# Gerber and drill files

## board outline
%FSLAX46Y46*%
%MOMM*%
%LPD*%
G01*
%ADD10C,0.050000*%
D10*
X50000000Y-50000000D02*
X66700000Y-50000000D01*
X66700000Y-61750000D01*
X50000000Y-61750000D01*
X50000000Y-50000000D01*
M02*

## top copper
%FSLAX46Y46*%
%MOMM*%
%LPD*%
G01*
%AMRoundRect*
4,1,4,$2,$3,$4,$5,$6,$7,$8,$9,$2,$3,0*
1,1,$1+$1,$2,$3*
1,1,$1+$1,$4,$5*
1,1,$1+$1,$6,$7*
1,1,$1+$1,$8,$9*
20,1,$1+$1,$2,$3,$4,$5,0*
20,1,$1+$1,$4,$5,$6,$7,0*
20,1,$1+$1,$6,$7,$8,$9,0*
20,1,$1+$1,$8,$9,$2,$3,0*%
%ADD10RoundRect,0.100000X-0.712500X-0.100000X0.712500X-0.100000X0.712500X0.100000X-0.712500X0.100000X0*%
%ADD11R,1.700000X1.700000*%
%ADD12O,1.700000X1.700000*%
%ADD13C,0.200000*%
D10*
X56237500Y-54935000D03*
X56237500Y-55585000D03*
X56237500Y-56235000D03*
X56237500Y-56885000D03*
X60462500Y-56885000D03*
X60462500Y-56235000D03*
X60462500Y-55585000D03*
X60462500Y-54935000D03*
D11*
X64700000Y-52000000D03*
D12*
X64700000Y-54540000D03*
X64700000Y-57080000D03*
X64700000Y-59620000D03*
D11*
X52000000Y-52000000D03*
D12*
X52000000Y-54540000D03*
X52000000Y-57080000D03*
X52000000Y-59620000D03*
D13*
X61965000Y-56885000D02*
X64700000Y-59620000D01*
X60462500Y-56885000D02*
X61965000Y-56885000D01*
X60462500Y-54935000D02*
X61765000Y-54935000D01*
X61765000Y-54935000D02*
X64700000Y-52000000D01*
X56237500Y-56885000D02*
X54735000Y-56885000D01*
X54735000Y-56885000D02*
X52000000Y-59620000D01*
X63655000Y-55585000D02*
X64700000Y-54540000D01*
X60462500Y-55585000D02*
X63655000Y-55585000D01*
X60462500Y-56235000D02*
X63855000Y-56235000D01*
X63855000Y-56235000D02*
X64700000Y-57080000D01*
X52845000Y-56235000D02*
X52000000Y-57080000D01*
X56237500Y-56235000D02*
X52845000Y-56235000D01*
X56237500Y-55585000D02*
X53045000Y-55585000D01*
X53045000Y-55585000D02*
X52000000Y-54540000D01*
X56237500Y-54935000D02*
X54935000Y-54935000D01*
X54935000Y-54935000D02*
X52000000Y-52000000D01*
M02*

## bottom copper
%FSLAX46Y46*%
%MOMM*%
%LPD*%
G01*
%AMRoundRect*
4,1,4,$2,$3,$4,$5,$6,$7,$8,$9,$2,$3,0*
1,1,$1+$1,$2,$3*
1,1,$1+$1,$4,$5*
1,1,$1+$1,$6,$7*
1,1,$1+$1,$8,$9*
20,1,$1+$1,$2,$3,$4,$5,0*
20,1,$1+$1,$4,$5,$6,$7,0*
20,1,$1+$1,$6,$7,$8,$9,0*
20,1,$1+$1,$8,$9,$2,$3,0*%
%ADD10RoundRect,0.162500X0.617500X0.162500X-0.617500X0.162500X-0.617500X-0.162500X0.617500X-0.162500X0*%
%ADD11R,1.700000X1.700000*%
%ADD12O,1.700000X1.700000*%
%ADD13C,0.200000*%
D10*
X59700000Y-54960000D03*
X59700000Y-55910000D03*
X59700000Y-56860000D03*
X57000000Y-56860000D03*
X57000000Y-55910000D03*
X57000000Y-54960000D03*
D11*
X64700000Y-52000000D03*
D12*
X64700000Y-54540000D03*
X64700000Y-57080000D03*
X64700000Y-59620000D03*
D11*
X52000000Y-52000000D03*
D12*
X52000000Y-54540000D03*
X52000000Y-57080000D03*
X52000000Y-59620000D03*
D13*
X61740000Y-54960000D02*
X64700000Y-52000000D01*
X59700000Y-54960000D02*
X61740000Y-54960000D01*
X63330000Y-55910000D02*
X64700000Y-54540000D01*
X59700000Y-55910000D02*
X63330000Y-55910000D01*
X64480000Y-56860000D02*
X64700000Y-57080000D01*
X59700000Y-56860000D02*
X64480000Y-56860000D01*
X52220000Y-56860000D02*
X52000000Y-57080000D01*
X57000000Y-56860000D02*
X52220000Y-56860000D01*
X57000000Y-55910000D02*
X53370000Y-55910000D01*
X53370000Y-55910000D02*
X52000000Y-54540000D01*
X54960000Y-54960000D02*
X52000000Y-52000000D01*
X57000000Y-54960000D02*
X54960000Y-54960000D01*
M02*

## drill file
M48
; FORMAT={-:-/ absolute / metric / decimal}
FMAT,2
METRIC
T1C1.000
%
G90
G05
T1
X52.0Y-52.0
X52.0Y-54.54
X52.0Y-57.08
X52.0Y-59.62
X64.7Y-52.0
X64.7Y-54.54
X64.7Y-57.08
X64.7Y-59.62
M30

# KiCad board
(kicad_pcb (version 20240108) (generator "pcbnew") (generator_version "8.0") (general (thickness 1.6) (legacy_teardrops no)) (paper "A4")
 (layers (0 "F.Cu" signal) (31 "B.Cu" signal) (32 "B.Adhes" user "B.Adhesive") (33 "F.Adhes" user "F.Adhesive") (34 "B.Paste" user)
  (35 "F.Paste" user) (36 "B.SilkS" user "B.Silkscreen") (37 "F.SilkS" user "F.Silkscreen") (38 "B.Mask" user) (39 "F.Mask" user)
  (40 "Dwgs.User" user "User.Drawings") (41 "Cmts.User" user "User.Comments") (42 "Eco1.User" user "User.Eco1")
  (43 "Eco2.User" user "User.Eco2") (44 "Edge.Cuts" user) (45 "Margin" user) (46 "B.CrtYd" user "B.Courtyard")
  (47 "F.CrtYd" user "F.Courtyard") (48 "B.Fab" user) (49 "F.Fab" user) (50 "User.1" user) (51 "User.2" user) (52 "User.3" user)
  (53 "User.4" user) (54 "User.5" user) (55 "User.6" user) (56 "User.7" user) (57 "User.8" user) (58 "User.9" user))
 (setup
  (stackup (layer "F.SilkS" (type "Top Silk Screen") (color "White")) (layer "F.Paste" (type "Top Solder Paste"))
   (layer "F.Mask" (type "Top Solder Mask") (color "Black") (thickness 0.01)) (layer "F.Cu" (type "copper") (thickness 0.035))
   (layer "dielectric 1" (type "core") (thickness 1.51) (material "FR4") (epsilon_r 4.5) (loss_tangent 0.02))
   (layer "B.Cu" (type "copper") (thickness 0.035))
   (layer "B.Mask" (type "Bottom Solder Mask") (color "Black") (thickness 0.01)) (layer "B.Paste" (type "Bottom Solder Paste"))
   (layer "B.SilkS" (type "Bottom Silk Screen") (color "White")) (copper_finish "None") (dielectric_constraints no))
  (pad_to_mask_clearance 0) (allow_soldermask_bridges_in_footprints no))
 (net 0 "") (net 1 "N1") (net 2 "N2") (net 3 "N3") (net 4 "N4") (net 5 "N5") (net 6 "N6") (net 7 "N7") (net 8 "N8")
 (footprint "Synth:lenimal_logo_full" (layer "F.Cu") (at 58.35 59)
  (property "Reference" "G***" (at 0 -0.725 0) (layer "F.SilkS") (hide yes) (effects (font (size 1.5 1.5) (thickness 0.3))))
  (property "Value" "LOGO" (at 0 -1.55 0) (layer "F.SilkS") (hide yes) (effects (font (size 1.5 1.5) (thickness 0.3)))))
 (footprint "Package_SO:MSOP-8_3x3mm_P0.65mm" (layer "F.Cu") (at 58.35 55.91)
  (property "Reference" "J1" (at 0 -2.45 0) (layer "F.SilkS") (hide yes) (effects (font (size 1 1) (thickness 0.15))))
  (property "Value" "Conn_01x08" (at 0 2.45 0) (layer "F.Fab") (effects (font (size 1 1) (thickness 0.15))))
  (pad "1" smd roundrect (at -2.1125 -0.975) (size 1.625 0.4) (layers "F.Cu" "F.Paste" "F.Mask") (roundrect_rratio 0.25) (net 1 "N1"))
  (pad "2" smd roundrect (at -2.1125 -0.325) (size 1.625 0.4) (layers "F.Cu" "F.Paste" "F.Mask") (roundrect_rratio 0.25) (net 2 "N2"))
  (pad "3" smd roundrect (at -2.1125 0.325) (size 1.625 0.4) (layers "F.Cu" "F.Paste" "F.Mask") (roundrect_rratio 0.25) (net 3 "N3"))
  (pad "4" smd roundrect (at -2.1125 0.975) (size 1.625 0.4) (layers "F.Cu" "F.Paste" "F.Mask") (roundrect_rratio 0.25) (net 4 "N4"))
  (pad "5" smd roundrect (at 2.1125 0.975) (size 1.625 0.4) (layers "F.Cu" "F.Paste" "F.Mask") (roundrect_rratio 0.25) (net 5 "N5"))
  (pad "6" smd roundrect (at 2.1125 0.325) (size 1.625 0.4) (layers "F.Cu" "F.Paste" "F.Mask") (roundrect_rratio 0.25) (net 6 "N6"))
  (pad "7" smd roundrect (at 2.1125 -0.325) (size 1.625 0.4) (layers "F.Cu" "F.Paste" "F.Mask") (roundrect_rratio 0.25) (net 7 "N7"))
  (pad "8" smd roundrect (at 2.1125 -0.975) (size 1.625 0.4) (layers "F.Cu" "F.Paste" "F.Mask") (roundrect_rratio 0.25) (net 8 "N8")))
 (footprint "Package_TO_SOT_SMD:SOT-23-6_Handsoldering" (layer "B.Cu") (at 58.35 55.91 180)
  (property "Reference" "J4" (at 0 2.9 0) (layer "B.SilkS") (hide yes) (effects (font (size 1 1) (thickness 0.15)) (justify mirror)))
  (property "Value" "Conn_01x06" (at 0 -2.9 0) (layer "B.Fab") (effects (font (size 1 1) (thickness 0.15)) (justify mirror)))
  (pad "1" smd roundrect (at -1.35 0.95 180) (size 1.56 0.65) (layers "B.Cu" "B.Paste" "B.Mask") (roundrect_rratio 0.25) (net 8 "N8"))
  (pad "2" smd roundrect (at -1.35 0 180) (size 1.56 0.65) (layers "B.Cu" "B.Paste" "B.Mask") (roundrect_rratio 0.25) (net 7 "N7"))
  (pad "3" smd roundrect (at -1.35 -0.95 180) (size 1.56 0.65) (layers "B.Cu" "B.Paste" "B.Mask") (roundrect_rratio 0.25) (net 6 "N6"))
  (pad "4" smd roundrect (at 1.35 -0.95 180) (size 1.56 0.65) (layers "B.Cu" "B.Paste" "B.Mask") (roundrect_rratio 0.25) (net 3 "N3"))
  (pad "5" smd roundrect (at 1.35 0 180) (size 1.56 0.65) (layers "B.Cu" "B.Paste" "B.Mask") (roundrect_rratio 0.25) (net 2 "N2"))
  (pad "6" smd roundrect (at 1.35 0.95 180) (size 1.56 0.65) (layers "B.Cu" "B.Paste" "B.Mask") (roundrect_rratio 0.25) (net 1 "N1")))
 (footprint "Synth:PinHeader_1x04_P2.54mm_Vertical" (layer "B.Cu") (at 64.7 52 180)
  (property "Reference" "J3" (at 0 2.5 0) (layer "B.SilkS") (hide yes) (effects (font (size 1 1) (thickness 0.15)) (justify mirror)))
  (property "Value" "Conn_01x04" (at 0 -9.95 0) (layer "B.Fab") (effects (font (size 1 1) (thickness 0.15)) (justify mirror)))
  (pad "1" thru_hole rect (at 0 0 180) (size 1.7 1.7) (drill 1) (layers "*.Cu" "*.Mask") (remove_unused_layers no) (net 8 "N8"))
  (pad "2" thru_hole oval (at 0 -2.54 180) (size 1.7 1.7) (drill 1) (layers "*.Cu" "*.Mask") (remove_unused_layers no) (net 7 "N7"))
  (pad "3" thru_hole oval (at 0 -5.08 180) (size 1.7 1.7) (drill 1) (layers "*.Cu" "*.Mask") (remove_unused_layers no) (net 6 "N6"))
  (pad "4" thru_hole oval (at 0 -7.62 180) (size 1.7 1.7) (drill 1) (layers "*.Cu" "*.Mask") (remove_unused_layers no) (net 5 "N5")))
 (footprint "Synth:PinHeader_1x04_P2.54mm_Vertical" (layer "B.Cu") (at 52 52 180)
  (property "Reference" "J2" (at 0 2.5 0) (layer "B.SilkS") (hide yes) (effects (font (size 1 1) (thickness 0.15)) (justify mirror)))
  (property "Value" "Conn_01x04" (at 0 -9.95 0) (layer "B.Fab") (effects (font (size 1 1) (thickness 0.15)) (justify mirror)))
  (pad "1" thru_hole rect (at 0 0 180) (size 1.7 1.7) (drill 1) (layers "*.Cu" "*.Mask") (remove_unused_layers no) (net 1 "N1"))
  (pad "2" thru_hole oval (at 0 -2.54 180) (size 1.7 1.7) (drill 1) (layers "*.Cu" "*.Mask") (remove_unused_layers no) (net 2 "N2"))
  (pad "3" thru_hole oval (at 0 -5.08 180) (size 1.7 1.7) (drill 1) (layers "*.Cu" "*.Mask") (remove_unused_layers no) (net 3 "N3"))
  (pad "4" thru_hole oval (at 0 -7.62 180) (size 1.7 1.7) (drill 1) (layers "*.Cu" "*.Mask") (remove_unused_layers no) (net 4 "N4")))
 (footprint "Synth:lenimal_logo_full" (layer "B.Cu") (at 58.35 53 180)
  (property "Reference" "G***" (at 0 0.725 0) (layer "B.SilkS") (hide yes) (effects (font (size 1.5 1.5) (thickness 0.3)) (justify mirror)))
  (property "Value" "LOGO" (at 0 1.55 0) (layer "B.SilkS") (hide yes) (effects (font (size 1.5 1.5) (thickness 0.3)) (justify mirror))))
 (gr_rect (start 50 50) (end 66.7 61.75) (stroke (width 0.05) (type default)) (fill none) (layer "Edge.Cuts"))
 (segment (start 61.965 56.885) (end 64.7 59.62) (width 0.2) (layer "F.Cu") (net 5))
 (segment (start 60.4625 56.885) (end 61.965 56.885) (width 0.2) (layer "F.Cu") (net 5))
 (segment (start 60.4625 54.935) (end 61.765 54.935) (width 0.2) (layer "F.Cu") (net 8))
 (segment (start 61.765 54.935) (end 64.7 52) (width 0.2) (layer "F.Cu") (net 8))
 (segment (start 61.74 54.96) (end 64.7 52) (width 0.2) (layer "B.Cu") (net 8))
 (segment (start 59.7 54.96) (end 61.74 54.96) (width 0.2) (layer "B.Cu") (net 8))
 (segment (start 56.2375 56.885) (end 54.735 56.885) (width 0.2) (layer "F.Cu") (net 4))
 (segment (start 54.735 56.885) (end 52 59.62) (width 0.2) (layer "F.Cu") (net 4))
 (segment (start 63.655 55.585) (end 64.7 54.54) (width 0.2) (layer "F.Cu") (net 7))
 (segment (start 60.4625 55.585) (end 63.655 55.585) (width 0.2) (layer "F.Cu") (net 7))
 (segment (start 63.33 55.91) (end 64.7 54.54) (width 0.2) (layer "B.Cu") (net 7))
 (segment (start 59.7 55.91) (end 63.33 55.91) (width 0.2) (layer "B.Cu") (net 7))
 (segment (start 60.4625 56.235) (end 63.855 56.235) (width 0.2) (layer "F.Cu") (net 6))
 (segment (start 63.855 56.235) (end 64.7 57.08) (width 0.2) (layer "F.Cu") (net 6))
 (segment (start 64.48 56.86) (end 64.7 57.08) (width 0.2) (layer "B.Cu") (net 6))
 (segment (start 59.7 56.86) (end 64.48 56.86) (width 0.2) (layer "B.Cu") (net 6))
 (segment (start 52.845 56.235) (end 52 57.08) (width 0.2) (layer "F.Cu") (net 3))
 (segment (start 56.2375 56.235) (end 52.845 56.235) (width 0.2) (layer "F.Cu") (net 3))
 (segment (start 52.22 56.86) (end 52 57.08) (width 0.2) (layer "B.Cu") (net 3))
 (segment (start 57 56.86) (end 52.22 56.86) (width 0.2) (layer "B.Cu") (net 3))
 (segment (start 56.2375 55.585) (end 53.045 55.585) (width 0.2) (layer "F.Cu") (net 2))
 (segment (start 53.045 55.585) (end 52 54.54) (width 0.2) (layer "F.Cu") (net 2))
 (segment (start 57 55.91) (end 53.37 55.91) (width 0.2) (layer "B.Cu") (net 2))
 (segment (start 53.37 55.91) (end 52 54.54) (width 0.2) (layer "B.Cu") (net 2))
 (segment (start 56.2375 54.935) (end 54.935 54.935) (width 0.2) (layer "F.Cu") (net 1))
 (segment (start 54.935 54.935) (end 52 52) (width 0.2) (layer "F.Cu") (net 1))
 (segment (start 54.96 54.96) (end 52 52) (width 0.2) (layer "B.Cu") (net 1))
 (segment (start 57 54.96) (end 54.96 54.96) (width 0.2) (layer "B.Cu") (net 1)))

